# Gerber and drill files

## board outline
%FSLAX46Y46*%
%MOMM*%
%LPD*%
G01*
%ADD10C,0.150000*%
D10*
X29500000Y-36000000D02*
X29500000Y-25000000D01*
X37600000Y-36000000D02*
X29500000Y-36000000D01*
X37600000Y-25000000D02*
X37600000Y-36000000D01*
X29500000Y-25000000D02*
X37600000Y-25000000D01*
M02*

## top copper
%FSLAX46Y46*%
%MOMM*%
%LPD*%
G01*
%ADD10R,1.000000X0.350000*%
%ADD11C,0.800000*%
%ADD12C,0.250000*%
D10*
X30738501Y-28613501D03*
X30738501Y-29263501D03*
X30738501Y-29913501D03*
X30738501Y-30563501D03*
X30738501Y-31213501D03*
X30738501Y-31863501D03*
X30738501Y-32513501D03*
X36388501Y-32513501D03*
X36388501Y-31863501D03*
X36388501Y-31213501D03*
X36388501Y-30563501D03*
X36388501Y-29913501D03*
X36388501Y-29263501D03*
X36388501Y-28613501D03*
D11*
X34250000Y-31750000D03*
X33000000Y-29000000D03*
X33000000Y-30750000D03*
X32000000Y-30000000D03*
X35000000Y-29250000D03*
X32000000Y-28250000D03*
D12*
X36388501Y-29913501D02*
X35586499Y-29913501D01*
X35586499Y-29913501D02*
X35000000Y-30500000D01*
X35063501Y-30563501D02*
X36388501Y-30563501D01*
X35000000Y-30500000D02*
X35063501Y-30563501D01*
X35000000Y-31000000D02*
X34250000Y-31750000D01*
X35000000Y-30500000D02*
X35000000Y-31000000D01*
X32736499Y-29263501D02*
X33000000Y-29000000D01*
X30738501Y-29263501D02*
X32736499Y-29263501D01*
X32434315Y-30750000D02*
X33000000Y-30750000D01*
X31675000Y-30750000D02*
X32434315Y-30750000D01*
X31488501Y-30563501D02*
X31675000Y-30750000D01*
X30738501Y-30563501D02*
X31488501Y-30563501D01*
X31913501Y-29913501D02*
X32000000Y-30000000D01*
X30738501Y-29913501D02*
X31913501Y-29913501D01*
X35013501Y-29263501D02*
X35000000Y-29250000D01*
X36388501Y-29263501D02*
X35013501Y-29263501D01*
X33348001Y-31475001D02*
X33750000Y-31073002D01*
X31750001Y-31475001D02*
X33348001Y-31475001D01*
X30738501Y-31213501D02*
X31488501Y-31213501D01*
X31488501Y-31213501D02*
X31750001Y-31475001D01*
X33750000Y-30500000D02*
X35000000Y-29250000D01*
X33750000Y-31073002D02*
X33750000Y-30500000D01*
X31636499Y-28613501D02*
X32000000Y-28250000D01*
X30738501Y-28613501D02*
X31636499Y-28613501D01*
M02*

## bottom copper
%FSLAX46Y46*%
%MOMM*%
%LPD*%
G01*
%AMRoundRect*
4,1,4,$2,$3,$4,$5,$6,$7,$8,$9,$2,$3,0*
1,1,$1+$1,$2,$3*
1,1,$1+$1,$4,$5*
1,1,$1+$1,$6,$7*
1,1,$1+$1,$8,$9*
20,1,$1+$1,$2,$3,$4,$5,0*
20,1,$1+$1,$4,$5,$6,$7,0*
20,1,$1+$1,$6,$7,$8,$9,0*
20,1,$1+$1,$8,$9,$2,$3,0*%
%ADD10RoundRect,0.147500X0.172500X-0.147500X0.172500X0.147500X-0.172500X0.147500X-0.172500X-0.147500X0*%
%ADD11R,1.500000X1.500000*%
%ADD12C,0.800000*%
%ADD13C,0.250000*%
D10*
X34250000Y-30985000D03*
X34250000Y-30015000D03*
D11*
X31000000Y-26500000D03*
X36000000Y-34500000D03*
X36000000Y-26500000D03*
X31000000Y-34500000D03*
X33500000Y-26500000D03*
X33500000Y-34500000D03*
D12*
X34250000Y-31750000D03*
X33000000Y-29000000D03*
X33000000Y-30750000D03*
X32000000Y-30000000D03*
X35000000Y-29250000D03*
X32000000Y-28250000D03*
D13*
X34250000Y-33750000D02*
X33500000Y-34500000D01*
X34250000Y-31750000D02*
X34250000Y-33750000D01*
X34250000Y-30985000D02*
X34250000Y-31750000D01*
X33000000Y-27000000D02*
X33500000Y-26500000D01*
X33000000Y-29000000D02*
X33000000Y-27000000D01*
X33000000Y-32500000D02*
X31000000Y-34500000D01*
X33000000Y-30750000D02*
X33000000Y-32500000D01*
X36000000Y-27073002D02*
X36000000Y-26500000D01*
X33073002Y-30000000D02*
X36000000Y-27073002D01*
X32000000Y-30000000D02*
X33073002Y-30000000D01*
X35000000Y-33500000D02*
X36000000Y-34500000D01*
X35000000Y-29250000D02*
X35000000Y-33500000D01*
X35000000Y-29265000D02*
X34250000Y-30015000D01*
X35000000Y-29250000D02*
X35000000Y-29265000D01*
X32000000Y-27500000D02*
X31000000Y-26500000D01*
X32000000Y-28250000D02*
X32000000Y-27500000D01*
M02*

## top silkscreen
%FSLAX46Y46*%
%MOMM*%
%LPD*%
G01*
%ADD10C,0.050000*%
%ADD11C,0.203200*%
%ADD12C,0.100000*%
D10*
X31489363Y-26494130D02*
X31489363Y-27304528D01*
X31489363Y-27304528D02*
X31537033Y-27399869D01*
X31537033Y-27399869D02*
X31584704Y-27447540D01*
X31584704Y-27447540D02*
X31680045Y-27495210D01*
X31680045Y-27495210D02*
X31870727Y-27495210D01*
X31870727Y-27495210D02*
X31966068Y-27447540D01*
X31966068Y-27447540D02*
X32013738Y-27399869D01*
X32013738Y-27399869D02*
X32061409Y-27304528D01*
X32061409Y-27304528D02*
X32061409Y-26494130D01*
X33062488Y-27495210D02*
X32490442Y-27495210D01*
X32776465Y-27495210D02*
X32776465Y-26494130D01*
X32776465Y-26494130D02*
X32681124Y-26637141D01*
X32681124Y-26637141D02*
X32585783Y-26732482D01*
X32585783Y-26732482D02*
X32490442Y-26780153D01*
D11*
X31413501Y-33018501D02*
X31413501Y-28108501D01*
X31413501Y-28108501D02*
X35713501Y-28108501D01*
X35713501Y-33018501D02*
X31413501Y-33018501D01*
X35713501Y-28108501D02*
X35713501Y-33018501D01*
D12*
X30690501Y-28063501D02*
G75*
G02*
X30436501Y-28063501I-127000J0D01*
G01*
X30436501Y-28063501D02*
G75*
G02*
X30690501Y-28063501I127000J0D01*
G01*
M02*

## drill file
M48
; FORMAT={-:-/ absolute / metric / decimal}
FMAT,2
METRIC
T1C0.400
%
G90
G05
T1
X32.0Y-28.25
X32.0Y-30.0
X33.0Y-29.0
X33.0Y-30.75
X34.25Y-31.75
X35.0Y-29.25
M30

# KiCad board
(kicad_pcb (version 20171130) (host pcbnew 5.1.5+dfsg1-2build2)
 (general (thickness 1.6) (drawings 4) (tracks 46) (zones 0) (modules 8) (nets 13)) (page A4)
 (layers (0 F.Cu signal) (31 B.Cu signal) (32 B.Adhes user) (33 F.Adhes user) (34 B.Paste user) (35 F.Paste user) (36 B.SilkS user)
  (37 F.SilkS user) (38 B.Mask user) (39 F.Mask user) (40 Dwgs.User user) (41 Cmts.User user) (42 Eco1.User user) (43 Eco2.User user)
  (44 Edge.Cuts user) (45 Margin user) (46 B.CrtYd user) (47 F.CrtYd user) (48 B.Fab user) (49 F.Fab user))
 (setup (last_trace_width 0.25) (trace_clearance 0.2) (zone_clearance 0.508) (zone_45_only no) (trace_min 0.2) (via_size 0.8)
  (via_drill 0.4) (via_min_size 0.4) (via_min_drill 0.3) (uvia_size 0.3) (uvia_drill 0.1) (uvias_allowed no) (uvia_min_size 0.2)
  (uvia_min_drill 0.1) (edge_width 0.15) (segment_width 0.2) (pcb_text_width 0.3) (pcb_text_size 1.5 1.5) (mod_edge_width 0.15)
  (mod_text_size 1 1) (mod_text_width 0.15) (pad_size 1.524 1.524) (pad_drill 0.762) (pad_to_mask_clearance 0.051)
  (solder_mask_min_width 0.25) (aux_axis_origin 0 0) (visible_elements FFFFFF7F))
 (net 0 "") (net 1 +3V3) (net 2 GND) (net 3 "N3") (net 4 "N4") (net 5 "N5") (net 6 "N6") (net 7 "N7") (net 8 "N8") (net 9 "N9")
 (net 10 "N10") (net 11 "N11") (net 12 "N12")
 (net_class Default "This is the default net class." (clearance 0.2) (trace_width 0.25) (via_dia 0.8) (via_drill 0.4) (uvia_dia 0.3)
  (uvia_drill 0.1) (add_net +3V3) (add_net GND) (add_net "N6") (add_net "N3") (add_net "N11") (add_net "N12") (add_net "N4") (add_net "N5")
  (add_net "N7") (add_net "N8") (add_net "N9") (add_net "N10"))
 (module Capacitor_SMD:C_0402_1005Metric (layer B.Cu) (at 34.25 30.5 90)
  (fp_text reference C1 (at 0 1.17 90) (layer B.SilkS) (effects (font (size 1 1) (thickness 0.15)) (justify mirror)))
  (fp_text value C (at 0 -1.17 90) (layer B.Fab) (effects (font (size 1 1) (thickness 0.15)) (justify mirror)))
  (pad 1 smd roundrect (at -0.485 0 90) (size 0.59 0.64) (layers B.Cu B.Paste B.Mask) (roundrect_rratio 0.25) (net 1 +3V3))
  (pad 2 smd roundrect (at 0.485 0 90) (size 0.59 0.64) (layers B.Cu B.Paste B.Mask) (roundrect_rratio 0.25) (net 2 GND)))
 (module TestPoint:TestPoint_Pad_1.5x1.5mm (layer B.Cu) (at 31 26.5)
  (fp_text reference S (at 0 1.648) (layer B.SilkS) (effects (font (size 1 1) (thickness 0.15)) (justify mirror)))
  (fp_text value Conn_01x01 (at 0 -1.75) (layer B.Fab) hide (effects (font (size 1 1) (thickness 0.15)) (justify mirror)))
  (pad 1 smd rect (at 0 0) (size 1.5 1.5) (layers B.Cu B.Mask) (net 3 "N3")))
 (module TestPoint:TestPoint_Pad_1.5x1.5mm (layer B.Cu) (at 36 34.5 180)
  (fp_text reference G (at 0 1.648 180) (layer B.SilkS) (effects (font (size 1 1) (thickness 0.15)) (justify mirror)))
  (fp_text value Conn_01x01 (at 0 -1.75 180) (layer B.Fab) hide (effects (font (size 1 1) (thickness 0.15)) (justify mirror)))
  (pad 1 smd rect (at 0 0 180) (size 1.5 1.5) (layers B.Cu B.Mask) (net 2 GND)))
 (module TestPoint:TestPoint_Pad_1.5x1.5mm (layer B.Cu) (at 36 26.5)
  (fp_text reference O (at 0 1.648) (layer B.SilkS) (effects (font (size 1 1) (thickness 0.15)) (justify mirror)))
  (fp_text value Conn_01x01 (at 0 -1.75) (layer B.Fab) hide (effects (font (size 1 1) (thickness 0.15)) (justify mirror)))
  (pad 1 smd rect (at 0 0) (size 1.5 1.5) (layers B.Cu B.Mask) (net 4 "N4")))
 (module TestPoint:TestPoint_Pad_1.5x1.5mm (layer B.Cu) (at 31 34.5 180)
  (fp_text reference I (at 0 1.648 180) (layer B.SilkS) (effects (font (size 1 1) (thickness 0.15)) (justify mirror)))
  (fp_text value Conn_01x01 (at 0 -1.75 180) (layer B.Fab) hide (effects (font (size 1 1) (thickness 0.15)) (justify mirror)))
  (pad 1 smd rect (at 0 0 180) (size 1.5 1.5) (layers B.Cu B.Mask) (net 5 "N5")))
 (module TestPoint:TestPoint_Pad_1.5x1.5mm (layer B.Cu) (at 33.5 26.5)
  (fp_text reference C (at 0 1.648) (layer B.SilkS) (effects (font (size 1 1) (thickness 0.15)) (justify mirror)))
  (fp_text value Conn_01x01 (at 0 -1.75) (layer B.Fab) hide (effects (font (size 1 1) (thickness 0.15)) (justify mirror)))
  (pad 1 smd rect (at 0 0) (size 1.5 1.5) (layers B.Cu B.Mask) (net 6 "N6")))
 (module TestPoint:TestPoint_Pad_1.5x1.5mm (layer B.Cu) (at 33.5 34.5 180)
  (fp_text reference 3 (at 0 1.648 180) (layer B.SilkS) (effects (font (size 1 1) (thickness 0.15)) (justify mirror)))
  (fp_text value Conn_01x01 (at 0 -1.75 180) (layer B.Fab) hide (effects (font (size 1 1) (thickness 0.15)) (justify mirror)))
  (pad 1 smd rect (at 0 0 180) (size 1.5 1.5) (layers B.Cu B.Mask) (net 1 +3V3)))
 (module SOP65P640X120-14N (layer F.Cu) (at 33.563501 30.563501)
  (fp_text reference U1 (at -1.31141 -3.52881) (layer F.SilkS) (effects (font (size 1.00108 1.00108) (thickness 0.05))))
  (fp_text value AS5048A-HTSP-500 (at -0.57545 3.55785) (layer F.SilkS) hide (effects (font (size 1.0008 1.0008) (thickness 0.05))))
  (fp_line (start -2.15 2.455) (end -2.15 -2.455) (layer F.SilkS) (width 0.2032))
  (fp_line (start -2.15 -2.455) (end 2.15 -2.455) (layer F.SilkS) (width 0.2032))
  (fp_line (start 2.15 2.455) (end -2.15 2.455) (layer F.SilkS) (width 0.2032))
  (fp_line (start 2.15 -2.455) (end 2.15 2.455) (layer F.SilkS) (width 0.2032))
  (fp_circle (center -3 -2.5) (end -2.873 -2.5) (layer F.SilkS) (width 0.1))
  (pad 1 smd rect (at -2.825 -1.95 270) (size 0.35 1) (layers F.Cu F.Paste F.Mask) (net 3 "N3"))
  (pad 2 smd rect (at -2.825 -1.3 270) (size 0.35 1) (layers F.Cu F.Paste F.Mask) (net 6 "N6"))
  (pad 3 smd rect (at -2.825 -0.65 270) (size 0.35 1) (layers F.Cu F.Paste F.Mask) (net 4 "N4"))
  (pad 4 smd rect (at -2.825 0 270) (size 0.35 1) (layers F.Cu F.Paste F.Mask) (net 5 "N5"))
  (pad 5 smd rect (at -2.825 0.65 270) (size 0.35 1) (layers F.Cu F.Paste F.Mask) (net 2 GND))
  (pad 6 smd rect (at -2.825 1.3 270) (size 0.35 1) (layers F.Cu F.Paste F.Mask) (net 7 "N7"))
  (pad 7 smd rect (at -2.825 1.95 270) (size 0.35 1) (layers F.Cu F.Paste F.Mask) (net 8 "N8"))
  (pad 8 smd rect (at 2.825 1.95 90) (size 0.35 1) (layers F.Cu F.Paste F.Mask) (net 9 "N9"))
  (pad 9 smd rect (at 2.825 1.3 90) (size 0.35 1) (layers F.Cu F.Paste F.Mask) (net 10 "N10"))
  (pad 10 smd rect (at 2.825 0.65 90) (size 0.35 1) (layers F.Cu F.Paste F.Mask) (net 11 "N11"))
  (pad 11 smd rect (at 2.825 0 90) (size 0.35 1) (layers F.Cu F.Paste F.Mask) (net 1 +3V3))
  (pad 12 smd rect (at 2.825 -0.65 90) (size 0.35 1) (layers F.Cu F.Paste F.Mask) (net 1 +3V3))
  (pad 13 smd rect (at 2.825 -1.3 90) (size 0.35 1) (layers F.Cu F.Paste F.Mask) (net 2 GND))
  (pad 14 smd rect (at 2.825 -1.95 90) (size 0.35 1) (layers F.Cu F.Paste F.Mask) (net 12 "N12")))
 (gr_line (start 29.5 36) (end 29.5 25) (layer Edge.Cuts) (width 0.15))
 (gr_line (start 37.6 36) (end 29.5 36) (layer Edge.Cuts) (width 0.15))
 (gr_line (start 37.6 25) (end 37.6 36) (layer Edge.Cuts) (width 0.15))
 (gr_line (start 29.5 25) (end 37.6 25) (layer Edge.Cuts) (width 0.15))
 (via (at 34.25 31.75) (size 0.8) (drill 0.4) (layers F.Cu B.Cu) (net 1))
 (segment (start 36.388501 29.913501) (end 35.586499 29.913501) (width 0.25) (layer F.Cu) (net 1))
 (segment (start 35.586499 29.913501) (end 35 30.5) (width 0.25) (layer F.Cu) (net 1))
 (segment (start 35.063501 30.563501) (end 36.388501 30.563501) (width 0.25) (layer F.Cu) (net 1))
 (segment (start 35 30.5) (end 35.063501 30.563501) (width 0.25) (layer F.Cu) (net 1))
 (segment (start 35 31) (end 34.25 31.75) (width 0.25) (layer F.Cu) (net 1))
 (segment (start 35 30.5) (end 35 31) (width 0.25) (layer F.Cu) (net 1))
 (segment (start 34.25 33.75) (end 33.5 34.5) (width 0.25) (layer B.Cu) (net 1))
 (segment (start 34.25 31.75) (end 34.25 33.75) (width 0.25) (layer B.Cu) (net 1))
 (segment (start 34.25 30.985) (end 34.25 31.75) (width 0.25) (layer B.Cu) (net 1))
 (via (at 33 29) (size 0.8) (drill 0.4) (layers F.Cu B.Cu) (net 6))
 (segment (start 32.736499 29.263501) (end 33 29) (width 0.25) (layer F.Cu) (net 6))
 (segment (start 30.738501 29.263501) (end 32.736499 29.263501) (width 0.25) (layer F.Cu) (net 6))
 (segment (start 33 27) (end 33.5 26.5) (width 0.25) (layer B.Cu) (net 6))
 (segment (start 33 29) (end 33 27) (width 0.25) (layer B.Cu) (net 6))
 (via (at 33 30.75) (size 0.8) (drill 0.4) (layers F.Cu B.Cu) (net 5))
 (segment (start 32.434315 30.75) (end 33 30.75) (width 0.25) (layer F.Cu) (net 5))
 (segment (start 31.675 30.75) (end 32.434315 30.75) (width 0.25) (layer F.Cu) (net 5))
 (segment (start 31.488501 30.563501) (end 31.675 30.75) (width 0.25) (layer F.Cu) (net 5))
 (segment (start 30.738501 30.563501) (end 31.488501 30.563501) (width 0.25) (layer F.Cu) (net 5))
 (segment (start 33 32.5) (end 31 34.5) (width 0.25) (layer B.Cu) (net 5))
 (segment (start 33 30.75) (end 33 32.5) (width 0.25) (layer B.Cu) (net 5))
 (via (at 32 30) (size 0.8) (drill 0.4) (layers F.Cu B.Cu) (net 4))
 (segment (start 31.913501 29.913501) (end 32 30) (width 0.25) (layer F.Cu) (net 4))
 (segment (start 30.738501 29.913501) (end 31.913501 29.913501) (width 0.25) (layer F.Cu) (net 4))
 (segment (start 36 27.073002) (end 36 26.5) (width 0.25) (layer B.Cu) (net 4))
 (segment (start 33.073002 30) (end 36 27.073002) (width 0.25) (layer B.Cu) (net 4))
 (segment (start 32 30) (end 33.073002 30) (width 0.25) (layer B.Cu) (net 4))
 (via (at 35 29.25) (size 0.8) (drill 0.4) (layers F.Cu B.Cu) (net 2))
 (segment (start 35.013501 29.263501) (end 35 29.25) (width 0.25) (layer F.Cu) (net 2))
 (segment (start 36.388501 29.263501) (end 35.013501 29.263501) (width 0.25) (layer F.Cu) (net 2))
 (segment (start 33.348001 31.475001) (end 33.75 31.073002) (width 0.25) (layer F.Cu) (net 2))
 (segment (start 31.750001 31.475001) (end 33.348001 31.475001) (width 0.25) (layer F.Cu) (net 2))
 (segment (start 30.738501 31.213501) (end 31.488501 31.213501) (width 0.25) (layer F.Cu) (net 2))
 (segment (start 31.488501 31.213501) (end 31.750001 31.475001) (width 0.25) (layer F.Cu) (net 2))
 (segment (start 33.75 30.5) (end 35 29.25) (width 0.25) (layer F.Cu) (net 2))
 (segment (start 33.75 31.073002) (end 33.75 30.5) (width 0.25) (layer F.Cu) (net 2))
 (segment (start 35 33.5) (end 36 34.5) (width 0.25) (layer B.Cu) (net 2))
 (segment (start 35 29.25) (end 35 33.5) (width 0.25) (layer B.Cu) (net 2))
 (segment (start 35 29.265) (end 34.25 30.015) (width 0.25) (layer B.Cu) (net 2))
 (segment (start 35 29.25) (end 35 29.265) (width 0.25) (layer B.Cu) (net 2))
 (via (at 32 28.25) (size 0.8) (drill 0.4) (layers F.Cu B.Cu) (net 3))
 (segment (start 31.636499 28.613501) (end 32 28.25) (width 0.25) (layer F.Cu) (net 3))
 (segment (start 30.738501 28.613501) (end 31.636499 28.613501) (width 0.25) (layer F.Cu) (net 3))
 (segment (start 32 27.5) (end 31 26.5) (width 0.25) (layer B.Cu) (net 3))
 (segment (start 32 28.25) (end 32 27.5) (width 0.25) (layer B.Cu) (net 3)))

